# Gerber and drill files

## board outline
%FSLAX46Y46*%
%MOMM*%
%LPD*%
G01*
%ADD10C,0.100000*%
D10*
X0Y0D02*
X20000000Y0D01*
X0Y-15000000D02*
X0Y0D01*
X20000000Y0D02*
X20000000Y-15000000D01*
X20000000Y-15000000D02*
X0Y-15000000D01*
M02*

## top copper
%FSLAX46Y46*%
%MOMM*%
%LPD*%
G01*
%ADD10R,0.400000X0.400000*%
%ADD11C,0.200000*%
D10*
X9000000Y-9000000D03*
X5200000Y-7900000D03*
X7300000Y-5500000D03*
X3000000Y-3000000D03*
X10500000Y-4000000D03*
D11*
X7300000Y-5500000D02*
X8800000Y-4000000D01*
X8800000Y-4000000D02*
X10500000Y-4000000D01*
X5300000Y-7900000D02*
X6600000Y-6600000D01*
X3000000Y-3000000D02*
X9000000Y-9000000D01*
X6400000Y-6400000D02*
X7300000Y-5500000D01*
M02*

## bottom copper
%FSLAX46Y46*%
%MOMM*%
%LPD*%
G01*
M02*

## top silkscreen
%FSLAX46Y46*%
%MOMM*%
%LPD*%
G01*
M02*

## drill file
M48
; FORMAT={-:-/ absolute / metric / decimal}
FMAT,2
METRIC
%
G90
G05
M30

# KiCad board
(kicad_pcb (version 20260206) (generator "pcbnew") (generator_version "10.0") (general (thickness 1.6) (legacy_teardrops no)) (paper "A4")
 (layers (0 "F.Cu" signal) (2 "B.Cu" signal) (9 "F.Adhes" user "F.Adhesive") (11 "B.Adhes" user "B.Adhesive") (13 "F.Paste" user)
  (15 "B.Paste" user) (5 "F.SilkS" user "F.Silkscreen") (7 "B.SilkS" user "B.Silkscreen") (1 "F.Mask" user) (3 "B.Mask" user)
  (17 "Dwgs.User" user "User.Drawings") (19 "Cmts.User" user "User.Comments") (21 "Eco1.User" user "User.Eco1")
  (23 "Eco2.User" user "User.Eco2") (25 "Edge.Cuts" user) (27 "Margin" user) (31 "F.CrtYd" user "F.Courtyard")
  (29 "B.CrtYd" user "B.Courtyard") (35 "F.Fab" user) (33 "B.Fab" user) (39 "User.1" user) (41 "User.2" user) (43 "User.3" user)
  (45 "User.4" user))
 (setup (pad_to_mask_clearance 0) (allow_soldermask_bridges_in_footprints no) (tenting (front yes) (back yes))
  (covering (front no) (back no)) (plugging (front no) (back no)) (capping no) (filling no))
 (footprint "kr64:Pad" (layer "F.Cu") (at 9 9)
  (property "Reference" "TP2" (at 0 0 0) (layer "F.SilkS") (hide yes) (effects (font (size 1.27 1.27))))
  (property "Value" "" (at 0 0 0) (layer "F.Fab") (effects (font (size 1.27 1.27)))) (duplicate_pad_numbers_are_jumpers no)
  (pad "1" smd rect (at 0 0) (size 0.4 0.4) (layers "F.Cu" "F.Mask" "F.Paste") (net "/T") (thermal_bridge_angle 45)))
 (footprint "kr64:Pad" (layer "F.Cu") (at 5.2 7.9)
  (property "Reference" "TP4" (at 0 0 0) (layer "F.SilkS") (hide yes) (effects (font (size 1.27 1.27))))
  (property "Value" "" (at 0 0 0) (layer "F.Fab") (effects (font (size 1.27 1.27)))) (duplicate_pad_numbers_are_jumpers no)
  (pad "1" smd rect (at 0 0) (size 0.4 0.4) (layers "F.Cu" "F.Mask" "F.Paste") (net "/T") (thermal_bridge_angle 45)))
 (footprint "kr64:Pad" (layer "F.Cu") (at 7.3 5.5)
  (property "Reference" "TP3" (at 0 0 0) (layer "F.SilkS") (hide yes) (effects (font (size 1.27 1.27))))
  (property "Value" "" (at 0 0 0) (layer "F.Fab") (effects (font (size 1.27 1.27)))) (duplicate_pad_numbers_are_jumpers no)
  (pad "1" smd rect (at 0 0) (size 0.4 0.4) (layers "F.Cu" "F.Mask" "F.Paste") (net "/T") (thermal_bridge_angle 45)))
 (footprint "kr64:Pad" (layer "F.Cu") (at 3 3)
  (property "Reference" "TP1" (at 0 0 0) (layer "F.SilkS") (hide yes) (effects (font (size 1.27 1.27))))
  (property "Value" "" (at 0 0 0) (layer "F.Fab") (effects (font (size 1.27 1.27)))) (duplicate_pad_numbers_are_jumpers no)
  (pad "1" smd rect (at 0 0) (size 0.4 0.4) (layers "F.Cu" "F.Mask" "F.Paste") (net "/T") (thermal_bridge_angle 45)))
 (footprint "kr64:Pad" (layer "F.Cu") (at 10.5 4)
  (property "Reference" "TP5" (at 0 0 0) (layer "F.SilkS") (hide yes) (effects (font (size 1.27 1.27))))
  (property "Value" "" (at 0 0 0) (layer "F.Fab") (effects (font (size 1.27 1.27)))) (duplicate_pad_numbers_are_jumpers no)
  (pad "1" smd rect (at 0 0) (size 0.4 0.4) (layers "F.Cu" "F.Mask" "F.Paste") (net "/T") (thermal_bridge_angle 45)))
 (gr_line (start 0 0) (end 20 0) (stroke (width 0.1) (type default)) (layer "Edge.Cuts"))
 (gr_line (start 0 15) (end 0 0) (stroke (width 0.1) (type default)) (layer "Edge.Cuts"))
 (gr_line (start 20 0) (end 20 15) (stroke (width 0.1) (type default)) (layer "Edge.Cuts"))
 (gr_line (start 20 15) (end 0 15) (stroke (width 0.1) (type default)) (layer "Edge.Cuts"))
 (segment (start 7.3 5.5) (end 8.8 4) (width 0.2) (layer "F.Cu") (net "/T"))
 (segment (start 8.8 4) (end 10.5 4) (width 0.2) (layer "F.Cu") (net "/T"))
 (segment (start 5.3 7.9) (end 6.6 6.6) (width 0.2) (layer "F.Cu") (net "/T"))
 (segment (start 3 3) (end 9 9) (width 0.2) (layer "F.Cu") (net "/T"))
 (segment (start 6.4 6.4) (end 7.3 5.5) (width 0.2) (layer "F.Cu") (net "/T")))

